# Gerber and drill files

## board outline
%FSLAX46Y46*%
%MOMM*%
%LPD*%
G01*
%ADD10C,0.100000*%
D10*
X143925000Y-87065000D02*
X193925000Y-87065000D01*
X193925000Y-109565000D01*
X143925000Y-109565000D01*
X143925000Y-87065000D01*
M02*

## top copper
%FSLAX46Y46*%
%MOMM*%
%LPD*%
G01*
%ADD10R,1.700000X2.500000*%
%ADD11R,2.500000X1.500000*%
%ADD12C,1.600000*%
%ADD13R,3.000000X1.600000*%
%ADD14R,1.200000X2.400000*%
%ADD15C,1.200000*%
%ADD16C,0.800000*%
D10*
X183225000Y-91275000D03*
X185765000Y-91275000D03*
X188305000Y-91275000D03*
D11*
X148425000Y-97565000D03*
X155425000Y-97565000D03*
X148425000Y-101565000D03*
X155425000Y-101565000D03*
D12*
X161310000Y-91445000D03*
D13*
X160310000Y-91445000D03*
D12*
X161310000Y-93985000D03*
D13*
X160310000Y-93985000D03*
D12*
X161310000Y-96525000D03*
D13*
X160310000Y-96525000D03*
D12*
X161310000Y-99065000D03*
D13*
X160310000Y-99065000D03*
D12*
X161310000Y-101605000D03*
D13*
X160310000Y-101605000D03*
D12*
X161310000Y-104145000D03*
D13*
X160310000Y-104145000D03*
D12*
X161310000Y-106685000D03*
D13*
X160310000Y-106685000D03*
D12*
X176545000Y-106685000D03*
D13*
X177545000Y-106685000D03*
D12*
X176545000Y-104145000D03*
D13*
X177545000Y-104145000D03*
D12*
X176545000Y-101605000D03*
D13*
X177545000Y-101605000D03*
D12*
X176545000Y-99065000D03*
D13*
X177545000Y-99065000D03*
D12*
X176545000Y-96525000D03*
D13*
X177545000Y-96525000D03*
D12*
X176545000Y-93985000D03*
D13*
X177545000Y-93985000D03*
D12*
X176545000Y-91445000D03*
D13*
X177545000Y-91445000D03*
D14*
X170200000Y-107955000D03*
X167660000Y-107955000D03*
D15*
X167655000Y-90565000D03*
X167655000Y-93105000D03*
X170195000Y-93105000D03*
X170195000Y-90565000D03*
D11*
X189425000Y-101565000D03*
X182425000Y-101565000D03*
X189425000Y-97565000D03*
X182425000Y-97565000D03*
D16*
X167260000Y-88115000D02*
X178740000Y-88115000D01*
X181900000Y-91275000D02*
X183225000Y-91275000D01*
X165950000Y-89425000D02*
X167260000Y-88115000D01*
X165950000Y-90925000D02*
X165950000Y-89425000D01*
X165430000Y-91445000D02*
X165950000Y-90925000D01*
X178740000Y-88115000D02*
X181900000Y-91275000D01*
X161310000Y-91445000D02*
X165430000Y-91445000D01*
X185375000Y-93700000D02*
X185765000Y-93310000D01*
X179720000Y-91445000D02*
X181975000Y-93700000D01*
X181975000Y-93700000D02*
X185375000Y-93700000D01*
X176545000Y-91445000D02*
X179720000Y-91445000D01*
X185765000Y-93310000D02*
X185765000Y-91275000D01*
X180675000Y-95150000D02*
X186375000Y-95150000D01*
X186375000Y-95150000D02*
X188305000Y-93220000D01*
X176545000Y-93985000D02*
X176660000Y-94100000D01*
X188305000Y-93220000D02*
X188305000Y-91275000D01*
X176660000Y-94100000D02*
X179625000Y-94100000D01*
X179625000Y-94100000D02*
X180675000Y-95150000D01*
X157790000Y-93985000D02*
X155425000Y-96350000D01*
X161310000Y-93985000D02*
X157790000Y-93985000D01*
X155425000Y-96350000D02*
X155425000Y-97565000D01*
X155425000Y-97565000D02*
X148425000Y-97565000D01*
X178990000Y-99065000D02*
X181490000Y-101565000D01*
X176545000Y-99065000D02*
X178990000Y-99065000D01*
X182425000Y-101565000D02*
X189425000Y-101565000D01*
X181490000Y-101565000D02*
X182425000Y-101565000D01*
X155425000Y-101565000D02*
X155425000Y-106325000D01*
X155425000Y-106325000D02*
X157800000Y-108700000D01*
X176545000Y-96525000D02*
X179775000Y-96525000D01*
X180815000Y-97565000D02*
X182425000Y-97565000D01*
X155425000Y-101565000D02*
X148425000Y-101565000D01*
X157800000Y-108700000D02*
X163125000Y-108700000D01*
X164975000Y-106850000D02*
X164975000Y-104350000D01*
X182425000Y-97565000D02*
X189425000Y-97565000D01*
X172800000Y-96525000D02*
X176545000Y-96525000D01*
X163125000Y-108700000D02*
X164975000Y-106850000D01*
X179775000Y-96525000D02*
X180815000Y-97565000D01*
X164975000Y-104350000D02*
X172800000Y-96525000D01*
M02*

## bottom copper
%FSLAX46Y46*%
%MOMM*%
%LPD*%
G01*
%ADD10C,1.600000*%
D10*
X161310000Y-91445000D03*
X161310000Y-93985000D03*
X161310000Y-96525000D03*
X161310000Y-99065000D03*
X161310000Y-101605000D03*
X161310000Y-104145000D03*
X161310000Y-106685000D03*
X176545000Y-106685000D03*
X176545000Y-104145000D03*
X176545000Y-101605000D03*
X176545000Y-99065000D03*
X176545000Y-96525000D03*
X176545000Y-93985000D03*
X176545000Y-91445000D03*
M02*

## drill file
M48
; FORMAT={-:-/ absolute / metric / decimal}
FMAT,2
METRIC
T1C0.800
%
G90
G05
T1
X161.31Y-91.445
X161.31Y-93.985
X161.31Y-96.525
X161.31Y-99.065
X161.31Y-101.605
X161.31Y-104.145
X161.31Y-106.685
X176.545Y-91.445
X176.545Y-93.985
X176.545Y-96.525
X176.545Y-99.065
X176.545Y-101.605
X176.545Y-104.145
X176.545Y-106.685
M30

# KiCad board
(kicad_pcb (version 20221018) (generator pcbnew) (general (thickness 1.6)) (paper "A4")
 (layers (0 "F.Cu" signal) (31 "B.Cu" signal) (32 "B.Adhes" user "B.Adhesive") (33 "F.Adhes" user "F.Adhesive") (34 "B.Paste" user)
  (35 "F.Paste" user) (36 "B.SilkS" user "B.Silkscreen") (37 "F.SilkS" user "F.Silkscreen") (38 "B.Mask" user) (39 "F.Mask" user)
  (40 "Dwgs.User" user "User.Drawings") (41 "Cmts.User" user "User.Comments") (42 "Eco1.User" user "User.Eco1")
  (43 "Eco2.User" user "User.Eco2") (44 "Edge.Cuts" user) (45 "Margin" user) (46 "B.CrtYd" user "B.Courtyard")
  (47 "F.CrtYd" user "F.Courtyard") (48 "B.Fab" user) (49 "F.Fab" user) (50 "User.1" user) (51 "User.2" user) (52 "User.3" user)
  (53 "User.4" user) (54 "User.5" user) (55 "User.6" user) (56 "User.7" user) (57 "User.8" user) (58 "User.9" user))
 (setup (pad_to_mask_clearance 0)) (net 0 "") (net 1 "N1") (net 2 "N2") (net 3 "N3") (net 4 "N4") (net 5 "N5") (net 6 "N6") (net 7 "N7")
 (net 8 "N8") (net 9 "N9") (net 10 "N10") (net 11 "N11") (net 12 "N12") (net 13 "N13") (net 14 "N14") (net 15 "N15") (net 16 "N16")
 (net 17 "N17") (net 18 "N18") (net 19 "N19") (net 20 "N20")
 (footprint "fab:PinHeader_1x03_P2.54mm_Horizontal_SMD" (layer "F.Cu") (at 183.225 91.275 90)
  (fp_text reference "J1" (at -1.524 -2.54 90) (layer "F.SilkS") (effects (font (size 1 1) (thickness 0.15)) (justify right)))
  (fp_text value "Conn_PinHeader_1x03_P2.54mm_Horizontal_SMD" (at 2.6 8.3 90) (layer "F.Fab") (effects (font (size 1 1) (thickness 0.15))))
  (pad "1" smd rect (at 0 0 90) (size 2.5 1.7) (layers "F.Cu" "F.Paste" "F.Mask") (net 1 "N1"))
  (pad "2" smd rect (at 0 2.54 90) (size 2.5 1.7) (layers "F.Cu" "F.Paste" "F.Mask") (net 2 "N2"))
  (pad "3" smd rect (at 0 5.08 90) (size 2.5 1.7) (layers "F.Cu" "F.Paste" "F.Mask") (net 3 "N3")))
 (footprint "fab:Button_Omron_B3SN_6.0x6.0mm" (layer "F.Cu") (at 151.925 99.565)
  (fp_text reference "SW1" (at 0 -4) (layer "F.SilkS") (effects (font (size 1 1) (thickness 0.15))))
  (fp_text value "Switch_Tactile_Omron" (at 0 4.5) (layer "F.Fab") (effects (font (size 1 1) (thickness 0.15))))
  (pad "1" smd rect (at -3.5 -2) (size 2.5 1.5) (layers "F.Cu" "F.Paste" "F.Mask") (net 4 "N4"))
  (pad "1" smd rect (at 3.5 -2) (size 2.5 1.5) (layers "F.Cu" "F.Paste" "F.Mask") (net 4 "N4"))
  (pad "2" smd rect (at -3.5 2) (size 2.5 1.5) (layers "F.Cu" "F.Paste" "F.Mask") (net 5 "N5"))
  (pad "2" smd rect (at 3.5 2) (size 2.5 1.5) (layers "F.Cu" "F.Paste" "F.Mask") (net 5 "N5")))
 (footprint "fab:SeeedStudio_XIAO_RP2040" (layer "F.Cu") (at 168.925 99.065)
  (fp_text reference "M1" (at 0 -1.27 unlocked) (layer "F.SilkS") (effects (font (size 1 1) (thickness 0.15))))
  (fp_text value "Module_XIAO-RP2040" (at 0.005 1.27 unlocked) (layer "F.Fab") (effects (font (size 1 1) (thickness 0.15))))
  (pad "1" thru_hole circle (at -7.615 -7.62) (size 1.6 1.6) (drill 0.8) (layers "*.Cu" "*.Mask") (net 1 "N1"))
  (pad "1" smd rect (at -7.615 -7.62) (size 3 1.6) (drill (offset -1 0)) (layers "F.Cu" "F.Paste" "F.Mask") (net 1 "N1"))
  (pad "2" thru_hole circle (at -7.615 -5.08) (size 1.6 1.6) (drill 0.8) (layers "*.Cu" "*.Mask") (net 4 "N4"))
  (pad "2" smd rect (at -7.615 -5.08) (size 3 1.6) (drill (offset -1 0)) (layers "F.Cu" "F.Paste" "F.Mask") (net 4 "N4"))
  (pad "3" thru_hole circle (at -7.615 -2.54) (size 1.6 1.6) (drill 0.8) (layers "*.Cu" "*.Mask") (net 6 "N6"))
  (pad "3" smd rect (at -7.615 -2.54) (size 3 1.6) (drill (offset -1 0)) (layers "F.Cu" "F.Paste" "F.Mask") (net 6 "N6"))
  (pad "4" thru_hole circle (at -7.615 0) (size 1.6 1.6) (drill 0.8) (layers "*.Cu" "*.Mask") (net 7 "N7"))
  (pad "4" smd rect (at -7.615 0) (size 3 1.6) (drill (offset -1 0)) (layers "F.Cu" "F.Paste" "F.Mask") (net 7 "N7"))
  (pad "5" thru_hole circle (at -7.615 2.54) (size 1.6 1.6) (drill 0.8) (layers "*.Cu" "*.Mask") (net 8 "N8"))
  (pad "5" smd rect (at -7.615 2.54) (size 3 1.6) (drill (offset -1 0)) (layers "F.Cu" "F.Paste" "F.Mask") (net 8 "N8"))
  (pad "6" thru_hole circle (at -7.615 5.08) (size 1.6 1.6) (drill 0.8) (layers "*.Cu" "*.Mask") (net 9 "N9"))
  (pad "6" smd rect (at -7.615 5.08) (size 3 1.6) (drill (offset -1 0)) (layers "F.Cu" "F.Paste" "F.Mask") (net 9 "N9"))
  (pad "7" thru_hole circle (at -7.615 7.62) (size 1.6 1.6) (drill 0.8) (layers "*.Cu" "*.Mask") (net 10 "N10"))
  (pad "7" smd rect (at -7.615 7.62) (size 3 1.6) (drill (offset -1 0)) (layers "F.Cu" "F.Paste" "F.Mask") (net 10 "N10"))
  (pad "8" thru_hole circle (at 7.62 7.62) (size 1.6 1.6) (drill 0.8) (layers "*.Cu" "*.Mask") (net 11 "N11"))
  (pad "8" smd rect (at 7.62 7.62) (size 3 1.6) (drill (offset 1 0)) (layers "F.Cu" "F.Paste" "F.Mask") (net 11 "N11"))
  (pad "9" thru_hole circle (at 7.62 5.08) (size 1.6 1.6) (drill 0.8) (layers "*.Cu" "*.Mask") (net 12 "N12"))
  (pad "9" smd rect (at 7.62 5.08) (size 3 1.6) (drill (offset 1 0)) (layers "F.Cu" "F.Paste" "F.Mask") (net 12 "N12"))
  (pad "10" thru_hole circle (at 7.62 2.54) (size 1.6 1.6) (drill 0.8) (layers "*.Cu" "*.Mask") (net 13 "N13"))
  (pad "10" smd rect (at 7.62 2.54) (size 3 1.6) (drill (offset 1 0)) (layers "F.Cu" "F.Paste" "F.Mask") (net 13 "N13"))
  (pad "11" thru_hole circle (at 7.62 0) (size 1.6 1.6) (drill 0.8) (layers "*.Cu" "*.Mask") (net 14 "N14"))
  (pad "11" smd rect (at 7.62 0) (size 3 1.6) (drill (offset 1 0)) (layers "F.Cu" "F.Paste" "F.Mask") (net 14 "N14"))
  (pad "12" thru_hole circle (at 7.62 -2.54) (size 1.6 1.6) (drill 0.8) (layers "*.Cu" "*.Mask") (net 5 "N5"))
  (pad "12" smd rect (at 7.62 -2.54) (size 3 1.6) (drill (offset 1 0)) (layers "F.Cu" "F.Paste" "F.Mask") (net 5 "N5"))
  (pad "13" thru_hole circle (at 7.62 -5.08) (size 1.6 1.6) (drill 0.8) (layers "*.Cu" "*.Mask") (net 3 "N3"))
  (pad "13" smd rect (at 7.62 -5.08) (size 3 1.6) (drill (offset 1 0)) (layers "F.Cu" "F.Paste" "F.Mask") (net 3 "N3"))
  (pad "14" thru_hole circle (at 7.62 -7.62) (size 1.6 1.6) (drill 0.8) (layers "*.Cu" "*.Mask") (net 2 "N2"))
  (pad "14" smd rect (at 7.62 -7.62) (size 3 1.6) (drill (offset 1 0)) (layers "F.Cu" "F.Paste" "F.Mask") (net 2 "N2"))
  (pad "15" smd rect (at 1.275 8.89 270) (size 2.4 1.2) (layers "F.Cu" "F.Paste" "F.Mask") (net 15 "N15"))
  (pad "16" smd rect (at -1.265 8.89 270) (size 2.4 1.2) (layers "F.Cu" "F.Paste" "F.Mask") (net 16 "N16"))
  (pad "17" smd circle (at -1.27 -8.5) (size 1.2 1.2) (layers "F.Cu" "F.Paste" "F.Mask") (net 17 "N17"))
  (pad "18" smd circle (at -1.27 -5.96) (size 1.2 1.2) (layers "F.Cu" "F.Paste" "F.Mask") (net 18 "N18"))
  (pad "19" smd circle (at 1.27 -5.96) (size 1.2 1.2) (layers "F.Cu" "F.Paste" "F.Mask") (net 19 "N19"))
  (pad "20" smd circle (at 1.27 -8.5) (size 1.2 1.2) (layers "F.Cu" "F.Paste" "F.Mask") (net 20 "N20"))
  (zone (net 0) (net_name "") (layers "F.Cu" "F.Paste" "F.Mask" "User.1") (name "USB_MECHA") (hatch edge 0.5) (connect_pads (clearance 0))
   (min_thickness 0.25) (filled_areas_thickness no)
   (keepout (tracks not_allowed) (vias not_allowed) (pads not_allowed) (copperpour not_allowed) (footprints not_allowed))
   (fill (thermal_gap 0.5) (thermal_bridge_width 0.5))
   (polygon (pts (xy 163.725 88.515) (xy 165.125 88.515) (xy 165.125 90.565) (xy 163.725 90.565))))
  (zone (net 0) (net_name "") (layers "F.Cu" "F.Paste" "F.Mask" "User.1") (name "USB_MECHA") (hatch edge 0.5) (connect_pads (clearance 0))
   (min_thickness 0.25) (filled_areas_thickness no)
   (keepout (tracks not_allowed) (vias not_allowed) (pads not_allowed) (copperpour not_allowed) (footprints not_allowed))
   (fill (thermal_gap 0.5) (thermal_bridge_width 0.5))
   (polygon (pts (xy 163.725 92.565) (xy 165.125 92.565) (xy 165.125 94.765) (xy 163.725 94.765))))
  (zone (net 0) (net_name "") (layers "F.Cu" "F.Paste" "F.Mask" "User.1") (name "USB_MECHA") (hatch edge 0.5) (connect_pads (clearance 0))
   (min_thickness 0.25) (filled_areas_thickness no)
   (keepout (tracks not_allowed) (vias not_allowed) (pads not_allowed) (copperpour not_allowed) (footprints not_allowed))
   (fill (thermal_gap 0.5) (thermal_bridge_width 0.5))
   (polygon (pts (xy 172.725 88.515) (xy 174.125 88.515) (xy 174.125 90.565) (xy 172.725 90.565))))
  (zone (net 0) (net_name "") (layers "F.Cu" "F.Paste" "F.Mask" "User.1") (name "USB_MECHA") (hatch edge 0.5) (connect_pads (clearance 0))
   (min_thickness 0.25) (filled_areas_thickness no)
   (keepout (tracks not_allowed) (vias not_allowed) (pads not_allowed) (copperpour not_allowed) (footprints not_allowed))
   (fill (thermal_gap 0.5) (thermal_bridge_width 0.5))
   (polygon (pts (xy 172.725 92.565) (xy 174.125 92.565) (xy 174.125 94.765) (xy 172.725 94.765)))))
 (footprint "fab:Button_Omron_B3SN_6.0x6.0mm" (layer "F.Cu") (at 185.925 99.565 180)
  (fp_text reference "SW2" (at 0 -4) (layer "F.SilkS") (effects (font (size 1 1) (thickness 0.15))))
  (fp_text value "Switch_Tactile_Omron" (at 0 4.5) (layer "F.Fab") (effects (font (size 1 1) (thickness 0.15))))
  (pad "1" smd rect (at -3.5 -2 180) (size 2.5 1.5) (layers "F.Cu" "F.Paste" "F.Mask") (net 14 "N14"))
  (pad "1" smd rect (at 3.5 -2 180) (size 2.5 1.5) (layers "F.Cu" "F.Paste" "F.Mask") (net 14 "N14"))
  (pad "2" smd rect (at -3.5 2 180) (size 2.5 1.5) (layers "F.Cu" "F.Paste" "F.Mask") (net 5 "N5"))
  (pad "2" smd rect (at 3.5 2 180) (size 2.5 1.5) (layers "F.Cu" "F.Paste" "F.Mask") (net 5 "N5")))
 (gr_rect (start 143.925 87.065) (end 193.925 109.565) (stroke (width 0.1) (type default)) (fill none) (layer "Edge.Cuts"))
 (segment (start 167.26 88.115) (end 178.74 88.115) (width 0.8) (layer "F.Cu") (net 1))
 (segment (start 181.9 91.275) (end 183.225 91.275) (width 0.8) (layer "F.Cu") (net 1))
 (segment (start 165.95 89.425) (end 167.26 88.115) (width 0.8) (layer "F.Cu") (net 1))
 (segment (start 165.95 90.925) (end 165.95 89.425) (width 0.8) (layer "F.Cu") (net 1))
 (segment (start 165.43 91.445) (end 165.95 90.925) (width 0.8) (layer "F.Cu") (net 1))
 (segment (start 178.74 88.115) (end 181.9 91.275) (width 0.8) (layer "F.Cu") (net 1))
 (segment (start 161.31 91.445) (end 165.43 91.445) (width 0.8) (layer "F.Cu") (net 1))
 (segment (start 185.375 93.7) (end 185.765 93.31) (width 0.8) (layer "F.Cu") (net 2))
 (segment (start 179.72 91.445) (end 181.975 93.7) (width 0.8) (layer "F.Cu") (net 2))
 (segment (start 181.975 93.7) (end 185.375 93.7) (width 0.8) (layer "F.Cu") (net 2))
 (segment (start 176.545 91.445) (end 179.72 91.445) (width 0.8) (layer "F.Cu") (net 2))
 (segment (start 185.765 93.31) (end 185.765 91.275) (width 0.8) (layer "F.Cu") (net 2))
 (segment (start 180.675 95.15) (end 186.375 95.15) (width 0.8) (layer "F.Cu") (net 3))
 (segment (start 186.375 95.15) (end 188.305 93.22) (width 0.8) (layer "F.Cu") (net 3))
 (segment (start 176.545 93.985) (end 176.66 94.1) (width 0.8) (layer "F.Cu") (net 3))
 (segment (start 188.305 93.22) (end 188.305 91.275) (width 0.8) (layer "F.Cu") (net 3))
 (segment (start 176.66 94.1) (end 179.625 94.1) (width 0.8) (layer "F.Cu") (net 3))
 (segment (start 179.625 94.1) (end 180.675 95.15) (width 0.8) (layer "F.Cu") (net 3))
 (segment (start 157.79 93.985) (end 155.425 96.35) (width 0.8) (layer "F.Cu") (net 4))
 (segment (start 161.31 93.985) (end 157.79 93.985) (width 0.8) (layer "F.Cu") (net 4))
 (segment (start 155.425 96.35) (end 155.425 97.565) (width 0.8) (layer "F.Cu") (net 4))
 (segment (start 155.425 97.565) (end 148.425 97.565) (width 0.8) (layer "F.Cu") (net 4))
 (segment (start 178.99 99.065) (end 181.49 101.565) (width 0.8) (layer "F.Cu") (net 14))
 (segment (start 176.545 99.065) (end 178.99 99.065) (width 0.8) (layer "F.Cu") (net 14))
 (segment (start 182.425 101.565) (end 189.425 101.565) (width 0.8) (layer "F.Cu") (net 14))
 (segment (start 181.49 101.565) (end 182.425 101.565) (width 0.8) (layer "F.Cu") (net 14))
 (segment (start 155.425 101.565) (end 155.425 106.325) (width 0.8) (layer "F.Cu") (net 5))
 (segment (start 155.425 106.325) (end 157.8 108.7) (width 0.8) (layer "F.Cu") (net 5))
 (segment (start 176.545 96.525) (end 179.775 96.525) (width 0.8) (layer "F.Cu") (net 5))
 (segment (start 180.815 97.565) (end 182.425 97.565) (width 0.8) (layer "F.Cu") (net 5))
 (segment (start 155.425 101.565) (end 148.425 101.565) (width 0.8) (layer "F.Cu") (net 5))
 (segment (start 157.8 108.7) (end 163.125 108.7) (width 0.8) (layer "F.Cu") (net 5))
 (segment (start 164.975 106.85) (end 164.975 104.35) (width 0.8) (layer "F.Cu") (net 5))
 (segment (start 182.425 97.565) (end 189.425 97.565) (width 0.8) (layer "F.Cu") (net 5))
 (segment (start 172.8 96.525) (end 176.545 96.525) (width 0.8) (layer "F.Cu") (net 5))
 (segment (start 163.125 108.7) (end 164.975 106.85) (width 0.8) (layer "F.Cu") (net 5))
 (segment (start 179.775 96.525) (end 180.815 97.565) (width 0.8) (layer "F.Cu") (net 5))
 (segment (start 164.975 104.35) (end 172.8 96.525) (width 0.8) (layer "F.Cu") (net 5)))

